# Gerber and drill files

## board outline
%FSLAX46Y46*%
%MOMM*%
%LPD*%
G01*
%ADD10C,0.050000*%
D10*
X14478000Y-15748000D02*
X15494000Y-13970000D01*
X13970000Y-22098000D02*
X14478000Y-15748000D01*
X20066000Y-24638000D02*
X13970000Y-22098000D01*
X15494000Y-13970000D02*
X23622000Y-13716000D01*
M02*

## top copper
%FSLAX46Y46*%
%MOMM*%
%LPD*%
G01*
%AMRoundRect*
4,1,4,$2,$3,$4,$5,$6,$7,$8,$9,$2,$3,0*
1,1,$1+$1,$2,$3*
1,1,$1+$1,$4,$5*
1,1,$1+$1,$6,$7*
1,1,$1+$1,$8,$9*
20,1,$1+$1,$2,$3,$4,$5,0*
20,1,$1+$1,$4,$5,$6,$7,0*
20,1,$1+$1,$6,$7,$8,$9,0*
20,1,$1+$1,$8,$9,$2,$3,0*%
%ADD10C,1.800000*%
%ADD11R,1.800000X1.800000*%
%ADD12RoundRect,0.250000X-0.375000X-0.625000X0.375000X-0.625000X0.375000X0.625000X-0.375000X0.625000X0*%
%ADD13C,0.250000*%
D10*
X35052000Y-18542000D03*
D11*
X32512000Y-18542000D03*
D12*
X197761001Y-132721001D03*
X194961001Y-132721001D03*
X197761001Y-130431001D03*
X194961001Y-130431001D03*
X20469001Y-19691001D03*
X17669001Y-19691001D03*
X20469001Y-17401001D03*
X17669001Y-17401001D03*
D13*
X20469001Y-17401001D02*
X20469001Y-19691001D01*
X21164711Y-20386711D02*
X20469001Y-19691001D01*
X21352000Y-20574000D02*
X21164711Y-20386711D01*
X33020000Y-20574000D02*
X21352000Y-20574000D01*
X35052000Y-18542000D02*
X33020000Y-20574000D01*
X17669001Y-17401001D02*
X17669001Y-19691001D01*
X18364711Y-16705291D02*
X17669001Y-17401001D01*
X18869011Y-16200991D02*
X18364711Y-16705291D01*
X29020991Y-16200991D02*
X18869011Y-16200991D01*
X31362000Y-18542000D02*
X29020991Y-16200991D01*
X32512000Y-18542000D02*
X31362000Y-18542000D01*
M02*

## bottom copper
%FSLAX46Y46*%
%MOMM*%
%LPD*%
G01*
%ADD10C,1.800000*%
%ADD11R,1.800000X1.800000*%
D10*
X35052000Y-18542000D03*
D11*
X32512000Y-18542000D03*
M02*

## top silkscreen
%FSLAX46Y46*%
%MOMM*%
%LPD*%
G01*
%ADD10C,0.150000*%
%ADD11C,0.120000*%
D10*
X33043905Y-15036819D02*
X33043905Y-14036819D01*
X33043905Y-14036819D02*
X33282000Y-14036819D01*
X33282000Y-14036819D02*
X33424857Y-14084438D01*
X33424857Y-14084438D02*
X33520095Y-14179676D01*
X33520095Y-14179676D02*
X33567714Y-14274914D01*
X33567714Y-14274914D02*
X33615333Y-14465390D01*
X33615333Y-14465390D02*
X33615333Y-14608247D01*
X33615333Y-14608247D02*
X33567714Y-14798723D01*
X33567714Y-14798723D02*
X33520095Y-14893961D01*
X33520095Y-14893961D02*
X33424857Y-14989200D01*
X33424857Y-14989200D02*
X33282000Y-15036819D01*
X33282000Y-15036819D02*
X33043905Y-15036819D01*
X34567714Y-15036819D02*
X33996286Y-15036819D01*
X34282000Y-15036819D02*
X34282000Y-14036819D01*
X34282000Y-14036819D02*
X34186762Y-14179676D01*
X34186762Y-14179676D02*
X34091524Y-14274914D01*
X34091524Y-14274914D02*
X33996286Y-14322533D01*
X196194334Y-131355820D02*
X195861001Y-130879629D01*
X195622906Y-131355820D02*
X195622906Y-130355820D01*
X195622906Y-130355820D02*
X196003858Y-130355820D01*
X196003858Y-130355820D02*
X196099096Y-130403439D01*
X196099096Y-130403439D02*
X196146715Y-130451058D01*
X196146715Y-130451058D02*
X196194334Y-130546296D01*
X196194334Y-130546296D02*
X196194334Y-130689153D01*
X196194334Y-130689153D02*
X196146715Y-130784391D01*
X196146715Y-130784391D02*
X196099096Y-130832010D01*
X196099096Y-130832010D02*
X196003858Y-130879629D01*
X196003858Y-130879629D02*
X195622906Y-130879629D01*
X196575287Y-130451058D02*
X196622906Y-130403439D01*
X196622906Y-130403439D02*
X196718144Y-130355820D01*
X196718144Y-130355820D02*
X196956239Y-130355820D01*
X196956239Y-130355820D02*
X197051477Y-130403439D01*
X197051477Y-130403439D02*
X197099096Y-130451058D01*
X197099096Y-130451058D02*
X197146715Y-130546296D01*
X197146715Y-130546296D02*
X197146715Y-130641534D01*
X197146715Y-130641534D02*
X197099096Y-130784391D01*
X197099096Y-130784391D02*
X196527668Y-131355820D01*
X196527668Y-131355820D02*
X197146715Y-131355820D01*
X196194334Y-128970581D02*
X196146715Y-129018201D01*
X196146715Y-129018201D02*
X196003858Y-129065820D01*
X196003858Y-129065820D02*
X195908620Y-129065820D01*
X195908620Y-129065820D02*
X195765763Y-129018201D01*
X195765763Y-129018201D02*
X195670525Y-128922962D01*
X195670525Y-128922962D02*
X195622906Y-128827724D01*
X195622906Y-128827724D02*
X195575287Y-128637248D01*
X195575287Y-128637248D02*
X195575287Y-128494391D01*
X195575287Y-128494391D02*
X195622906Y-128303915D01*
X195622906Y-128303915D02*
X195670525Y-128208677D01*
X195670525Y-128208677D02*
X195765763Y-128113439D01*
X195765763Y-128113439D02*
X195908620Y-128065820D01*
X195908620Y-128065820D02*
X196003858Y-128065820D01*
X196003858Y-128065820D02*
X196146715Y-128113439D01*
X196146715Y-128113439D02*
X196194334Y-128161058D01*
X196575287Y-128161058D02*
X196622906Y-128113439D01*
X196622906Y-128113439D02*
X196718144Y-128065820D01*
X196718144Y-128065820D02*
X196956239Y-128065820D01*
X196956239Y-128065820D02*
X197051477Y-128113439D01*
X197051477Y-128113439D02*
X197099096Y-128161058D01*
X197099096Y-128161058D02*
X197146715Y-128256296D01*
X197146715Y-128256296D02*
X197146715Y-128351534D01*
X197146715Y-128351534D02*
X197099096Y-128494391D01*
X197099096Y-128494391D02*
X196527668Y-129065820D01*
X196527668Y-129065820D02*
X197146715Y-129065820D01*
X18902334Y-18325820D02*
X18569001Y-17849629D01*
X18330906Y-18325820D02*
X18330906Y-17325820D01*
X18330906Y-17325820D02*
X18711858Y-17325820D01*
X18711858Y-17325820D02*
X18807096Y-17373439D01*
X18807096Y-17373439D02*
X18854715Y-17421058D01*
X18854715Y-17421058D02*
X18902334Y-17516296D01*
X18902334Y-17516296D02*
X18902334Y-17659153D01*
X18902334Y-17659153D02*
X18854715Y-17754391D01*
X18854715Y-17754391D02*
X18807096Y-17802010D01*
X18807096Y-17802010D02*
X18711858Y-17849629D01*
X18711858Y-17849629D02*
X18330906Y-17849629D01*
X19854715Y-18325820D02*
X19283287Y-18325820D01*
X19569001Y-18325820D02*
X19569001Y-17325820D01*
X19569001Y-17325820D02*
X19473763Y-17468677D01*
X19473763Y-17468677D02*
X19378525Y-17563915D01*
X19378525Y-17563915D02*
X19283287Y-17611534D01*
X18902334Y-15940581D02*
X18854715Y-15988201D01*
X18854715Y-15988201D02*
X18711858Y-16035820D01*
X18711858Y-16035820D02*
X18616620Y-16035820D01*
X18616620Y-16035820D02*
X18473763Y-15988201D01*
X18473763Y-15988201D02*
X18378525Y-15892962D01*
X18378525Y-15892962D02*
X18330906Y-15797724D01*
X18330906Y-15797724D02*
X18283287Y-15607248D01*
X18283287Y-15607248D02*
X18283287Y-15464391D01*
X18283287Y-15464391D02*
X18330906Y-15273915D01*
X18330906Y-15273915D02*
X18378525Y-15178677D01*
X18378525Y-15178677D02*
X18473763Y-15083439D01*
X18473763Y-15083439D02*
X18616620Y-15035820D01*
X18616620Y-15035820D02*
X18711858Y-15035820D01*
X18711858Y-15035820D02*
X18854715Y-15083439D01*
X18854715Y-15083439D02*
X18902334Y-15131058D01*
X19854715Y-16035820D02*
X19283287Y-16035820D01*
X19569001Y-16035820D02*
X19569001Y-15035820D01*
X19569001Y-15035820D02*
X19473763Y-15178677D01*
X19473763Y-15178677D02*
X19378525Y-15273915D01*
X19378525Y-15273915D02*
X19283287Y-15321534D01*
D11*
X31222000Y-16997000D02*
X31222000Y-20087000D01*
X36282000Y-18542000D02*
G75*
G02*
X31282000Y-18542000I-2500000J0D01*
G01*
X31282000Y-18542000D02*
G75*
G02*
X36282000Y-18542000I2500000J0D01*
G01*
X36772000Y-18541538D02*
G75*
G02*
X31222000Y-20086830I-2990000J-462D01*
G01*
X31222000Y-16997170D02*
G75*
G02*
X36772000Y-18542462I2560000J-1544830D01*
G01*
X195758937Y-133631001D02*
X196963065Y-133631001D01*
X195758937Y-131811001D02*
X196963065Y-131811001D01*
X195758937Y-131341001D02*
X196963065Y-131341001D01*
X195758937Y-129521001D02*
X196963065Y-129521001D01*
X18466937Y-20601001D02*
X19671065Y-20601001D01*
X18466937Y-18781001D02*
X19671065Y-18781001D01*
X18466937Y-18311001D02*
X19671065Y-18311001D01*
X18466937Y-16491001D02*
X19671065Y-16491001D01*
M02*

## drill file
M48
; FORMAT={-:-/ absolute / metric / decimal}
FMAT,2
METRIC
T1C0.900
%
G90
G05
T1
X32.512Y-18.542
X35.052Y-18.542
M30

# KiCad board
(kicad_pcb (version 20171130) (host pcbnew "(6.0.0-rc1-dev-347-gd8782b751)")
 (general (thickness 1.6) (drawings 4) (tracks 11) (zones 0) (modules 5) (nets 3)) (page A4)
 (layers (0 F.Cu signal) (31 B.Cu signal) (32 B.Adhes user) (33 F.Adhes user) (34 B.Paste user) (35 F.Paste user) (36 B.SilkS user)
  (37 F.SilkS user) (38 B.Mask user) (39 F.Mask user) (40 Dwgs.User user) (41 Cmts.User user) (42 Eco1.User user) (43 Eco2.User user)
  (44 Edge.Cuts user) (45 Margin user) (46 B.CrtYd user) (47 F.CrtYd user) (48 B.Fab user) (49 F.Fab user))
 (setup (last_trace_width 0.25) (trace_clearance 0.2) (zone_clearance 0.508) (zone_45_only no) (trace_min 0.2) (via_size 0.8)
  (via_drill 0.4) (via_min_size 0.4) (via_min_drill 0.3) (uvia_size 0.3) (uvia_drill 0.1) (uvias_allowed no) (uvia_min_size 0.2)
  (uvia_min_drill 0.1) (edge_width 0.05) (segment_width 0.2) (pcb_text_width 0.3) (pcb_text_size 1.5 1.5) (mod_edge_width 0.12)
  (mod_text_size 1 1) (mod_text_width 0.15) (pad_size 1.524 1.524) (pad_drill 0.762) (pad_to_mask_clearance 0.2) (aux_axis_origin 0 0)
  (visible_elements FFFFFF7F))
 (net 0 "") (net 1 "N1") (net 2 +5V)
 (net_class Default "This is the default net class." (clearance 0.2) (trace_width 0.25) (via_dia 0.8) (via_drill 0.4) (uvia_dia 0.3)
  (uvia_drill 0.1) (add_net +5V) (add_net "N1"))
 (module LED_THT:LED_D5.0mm (layer F.Cu) (at 32.512 18.542)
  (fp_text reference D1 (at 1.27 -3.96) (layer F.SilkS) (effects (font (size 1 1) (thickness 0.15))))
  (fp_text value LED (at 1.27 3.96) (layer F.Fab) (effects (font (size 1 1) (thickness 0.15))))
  (fp_line (start -1.29 -1.545) (end -1.29 1.545) (layer F.SilkS) (width 0.12))
  (fp_circle (center 1.27 0) (end 3.77 0) (layer F.SilkS) (width 0.12))
  (fp_arc (start 1.27 0) (end -1.29 1.54483) (angle -148.9) (layer F.SilkS) (width 0.12))
  (fp_arc (start 1.27 0) (end -1.29 -1.54483) (angle 148.9) (layer F.SilkS) (width 0.12))
  (pad 2 thru_hole circle (at 2.54 0) (size 1.8 1.8) (drill 0.9) (layers *.Cu *.Mask) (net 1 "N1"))
  (pad 1 thru_hole rect (at 0 0) (size 1.8 1.8) (drill 0.9) (layers *.Cu *.Mask) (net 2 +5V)))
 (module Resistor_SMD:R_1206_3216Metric (layer F.Cu) (at 196.361001 132.721001)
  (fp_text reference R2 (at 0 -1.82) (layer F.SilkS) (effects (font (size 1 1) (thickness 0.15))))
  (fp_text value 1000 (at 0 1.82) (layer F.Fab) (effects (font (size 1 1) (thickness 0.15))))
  (fp_line (start -0.602064 0.91) (end 0.602064 0.91) (layer F.SilkS) (width 0.12))
  (fp_line (start -0.602064 -0.91) (end 0.602064 -0.91) (layer F.SilkS) (width 0.12))
  (pad 2 smd roundrect (at 1.4 0) (size 1.25 1.75) (layers F.Cu F.Paste F.Mask) (roundrect_rratio 0.2) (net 1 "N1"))
  (pad 1 smd roundrect (at -1.4 0) (size 1.25 1.75) (layers F.Cu F.Paste F.Mask) (roundrect_rratio 0.2) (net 2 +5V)))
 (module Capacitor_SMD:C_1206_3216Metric (layer F.Cu) (at 196.361001 130.431001)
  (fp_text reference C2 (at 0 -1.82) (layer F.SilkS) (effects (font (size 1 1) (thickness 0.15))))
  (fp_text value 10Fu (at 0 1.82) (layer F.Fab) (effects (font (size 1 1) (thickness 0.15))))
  (fp_line (start -0.602064 0.91) (end 0.602064 0.91) (layer F.SilkS) (width 0.12))
  (fp_line (start -0.602064 -0.91) (end 0.602064 -0.91) (layer F.SilkS) (width 0.12))
  (pad 2 smd roundrect (at 1.4 0) (size 1.25 1.75) (layers F.Cu F.Paste F.Mask) (roundrect_rratio 0.2) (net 1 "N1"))
  (pad 1 smd roundrect (at -1.4 0) (size 1.25 1.75) (layers F.Cu F.Paste F.Mask) (roundrect_rratio 0.2) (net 2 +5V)))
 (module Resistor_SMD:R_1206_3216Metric (layer F.Cu) (at 19.069001 19.691001)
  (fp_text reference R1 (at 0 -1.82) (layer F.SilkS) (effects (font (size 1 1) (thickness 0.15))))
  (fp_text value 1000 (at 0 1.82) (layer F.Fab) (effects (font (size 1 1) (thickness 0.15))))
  (fp_line (start -0.602064 0.91) (end 0.602064 0.91) (layer F.SilkS) (width 0.12))
  (fp_line (start -0.602064 -0.91) (end 0.602064 -0.91) (layer F.SilkS) (width 0.12))
  (pad 2 smd roundrect (at 1.4 0) (size 1.25 1.75) (layers F.Cu F.Paste F.Mask) (roundrect_rratio 0.2) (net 1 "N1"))
  (pad 1 smd roundrect (at -1.4 0) (size 1.25 1.75) (layers F.Cu F.Paste F.Mask) (roundrect_rratio 0.2) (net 2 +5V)))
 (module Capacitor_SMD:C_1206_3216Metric (layer F.Cu) (at 19.069001 17.401001)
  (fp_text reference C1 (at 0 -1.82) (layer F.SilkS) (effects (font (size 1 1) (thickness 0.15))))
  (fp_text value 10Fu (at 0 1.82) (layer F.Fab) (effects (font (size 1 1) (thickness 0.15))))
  (fp_line (start -0.602064 0.91) (end 0.602064 0.91) (layer F.SilkS) (width 0.12))
  (fp_line (start -0.602064 -0.91) (end 0.602064 -0.91) (layer F.SilkS) (width 0.12))
  (pad 2 smd roundrect (at 1.4 0) (size 1.25 1.75) (layers F.Cu F.Paste F.Mask) (roundrect_rratio 0.2) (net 1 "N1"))
  (pad 1 smd roundrect (at -1.4 0) (size 1.25 1.75) (layers F.Cu F.Paste F.Mask) (roundrect_rratio 0.2) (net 2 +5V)))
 (gr_line (start 14.478 15.748) (end 15.494 13.97) (layer Edge.Cuts) (width 0.05))
 (gr_line (start 13.97 22.098) (end 14.478 15.748) (layer Edge.Cuts) (width 0.05))
 (gr_line (start 20.066 24.638) (end 13.97 22.098) (layer Edge.Cuts) (width 0.05))
 (gr_line (start 15.494 13.97) (end 23.622 13.716) (layer Edge.Cuts) (width 0.05))
 (segment (start 20.469001 17.401001) (end 20.469001 19.691001) (width 0.25) (layer F.Cu) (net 1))
 (segment (start 21.164711 20.386711) (end 20.469001 19.691001) (width 0.25) (layer F.Cu) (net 1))
 (segment (start 21.352 20.574) (end 21.164711 20.386711) (width 0.25) (layer F.Cu) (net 1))
 (segment (start 33.02 20.574) (end 21.352 20.574) (width 0.25) (layer F.Cu) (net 1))
 (segment (start 35.052 18.542) (end 33.02 20.574) (width 0.25) (layer F.Cu) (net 1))
 (segment (start 17.669001 17.401001) (end 17.669001 19.691001) (width 0.25) (layer F.Cu) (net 2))
 (segment (start 18.364711 16.705291) (end 17.669001 17.401001) (width 0.25) (layer F.Cu) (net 2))
 (segment (start 18.869011 16.200991) (end 18.364711 16.705291) (width 0.25) (layer F.Cu) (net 2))
 (segment (start 29.020991 16.200991) (end 18.869011 16.200991) (width 0.25) (layer F.Cu) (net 2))
 (segment (start 31.362 18.542) (end 29.020991 16.200991) (width 0.25) (layer F.Cu) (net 2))
 (segment (start 32.512 18.542) (end 31.362 18.542) (width 0.25) (layer F.Cu) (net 2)))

